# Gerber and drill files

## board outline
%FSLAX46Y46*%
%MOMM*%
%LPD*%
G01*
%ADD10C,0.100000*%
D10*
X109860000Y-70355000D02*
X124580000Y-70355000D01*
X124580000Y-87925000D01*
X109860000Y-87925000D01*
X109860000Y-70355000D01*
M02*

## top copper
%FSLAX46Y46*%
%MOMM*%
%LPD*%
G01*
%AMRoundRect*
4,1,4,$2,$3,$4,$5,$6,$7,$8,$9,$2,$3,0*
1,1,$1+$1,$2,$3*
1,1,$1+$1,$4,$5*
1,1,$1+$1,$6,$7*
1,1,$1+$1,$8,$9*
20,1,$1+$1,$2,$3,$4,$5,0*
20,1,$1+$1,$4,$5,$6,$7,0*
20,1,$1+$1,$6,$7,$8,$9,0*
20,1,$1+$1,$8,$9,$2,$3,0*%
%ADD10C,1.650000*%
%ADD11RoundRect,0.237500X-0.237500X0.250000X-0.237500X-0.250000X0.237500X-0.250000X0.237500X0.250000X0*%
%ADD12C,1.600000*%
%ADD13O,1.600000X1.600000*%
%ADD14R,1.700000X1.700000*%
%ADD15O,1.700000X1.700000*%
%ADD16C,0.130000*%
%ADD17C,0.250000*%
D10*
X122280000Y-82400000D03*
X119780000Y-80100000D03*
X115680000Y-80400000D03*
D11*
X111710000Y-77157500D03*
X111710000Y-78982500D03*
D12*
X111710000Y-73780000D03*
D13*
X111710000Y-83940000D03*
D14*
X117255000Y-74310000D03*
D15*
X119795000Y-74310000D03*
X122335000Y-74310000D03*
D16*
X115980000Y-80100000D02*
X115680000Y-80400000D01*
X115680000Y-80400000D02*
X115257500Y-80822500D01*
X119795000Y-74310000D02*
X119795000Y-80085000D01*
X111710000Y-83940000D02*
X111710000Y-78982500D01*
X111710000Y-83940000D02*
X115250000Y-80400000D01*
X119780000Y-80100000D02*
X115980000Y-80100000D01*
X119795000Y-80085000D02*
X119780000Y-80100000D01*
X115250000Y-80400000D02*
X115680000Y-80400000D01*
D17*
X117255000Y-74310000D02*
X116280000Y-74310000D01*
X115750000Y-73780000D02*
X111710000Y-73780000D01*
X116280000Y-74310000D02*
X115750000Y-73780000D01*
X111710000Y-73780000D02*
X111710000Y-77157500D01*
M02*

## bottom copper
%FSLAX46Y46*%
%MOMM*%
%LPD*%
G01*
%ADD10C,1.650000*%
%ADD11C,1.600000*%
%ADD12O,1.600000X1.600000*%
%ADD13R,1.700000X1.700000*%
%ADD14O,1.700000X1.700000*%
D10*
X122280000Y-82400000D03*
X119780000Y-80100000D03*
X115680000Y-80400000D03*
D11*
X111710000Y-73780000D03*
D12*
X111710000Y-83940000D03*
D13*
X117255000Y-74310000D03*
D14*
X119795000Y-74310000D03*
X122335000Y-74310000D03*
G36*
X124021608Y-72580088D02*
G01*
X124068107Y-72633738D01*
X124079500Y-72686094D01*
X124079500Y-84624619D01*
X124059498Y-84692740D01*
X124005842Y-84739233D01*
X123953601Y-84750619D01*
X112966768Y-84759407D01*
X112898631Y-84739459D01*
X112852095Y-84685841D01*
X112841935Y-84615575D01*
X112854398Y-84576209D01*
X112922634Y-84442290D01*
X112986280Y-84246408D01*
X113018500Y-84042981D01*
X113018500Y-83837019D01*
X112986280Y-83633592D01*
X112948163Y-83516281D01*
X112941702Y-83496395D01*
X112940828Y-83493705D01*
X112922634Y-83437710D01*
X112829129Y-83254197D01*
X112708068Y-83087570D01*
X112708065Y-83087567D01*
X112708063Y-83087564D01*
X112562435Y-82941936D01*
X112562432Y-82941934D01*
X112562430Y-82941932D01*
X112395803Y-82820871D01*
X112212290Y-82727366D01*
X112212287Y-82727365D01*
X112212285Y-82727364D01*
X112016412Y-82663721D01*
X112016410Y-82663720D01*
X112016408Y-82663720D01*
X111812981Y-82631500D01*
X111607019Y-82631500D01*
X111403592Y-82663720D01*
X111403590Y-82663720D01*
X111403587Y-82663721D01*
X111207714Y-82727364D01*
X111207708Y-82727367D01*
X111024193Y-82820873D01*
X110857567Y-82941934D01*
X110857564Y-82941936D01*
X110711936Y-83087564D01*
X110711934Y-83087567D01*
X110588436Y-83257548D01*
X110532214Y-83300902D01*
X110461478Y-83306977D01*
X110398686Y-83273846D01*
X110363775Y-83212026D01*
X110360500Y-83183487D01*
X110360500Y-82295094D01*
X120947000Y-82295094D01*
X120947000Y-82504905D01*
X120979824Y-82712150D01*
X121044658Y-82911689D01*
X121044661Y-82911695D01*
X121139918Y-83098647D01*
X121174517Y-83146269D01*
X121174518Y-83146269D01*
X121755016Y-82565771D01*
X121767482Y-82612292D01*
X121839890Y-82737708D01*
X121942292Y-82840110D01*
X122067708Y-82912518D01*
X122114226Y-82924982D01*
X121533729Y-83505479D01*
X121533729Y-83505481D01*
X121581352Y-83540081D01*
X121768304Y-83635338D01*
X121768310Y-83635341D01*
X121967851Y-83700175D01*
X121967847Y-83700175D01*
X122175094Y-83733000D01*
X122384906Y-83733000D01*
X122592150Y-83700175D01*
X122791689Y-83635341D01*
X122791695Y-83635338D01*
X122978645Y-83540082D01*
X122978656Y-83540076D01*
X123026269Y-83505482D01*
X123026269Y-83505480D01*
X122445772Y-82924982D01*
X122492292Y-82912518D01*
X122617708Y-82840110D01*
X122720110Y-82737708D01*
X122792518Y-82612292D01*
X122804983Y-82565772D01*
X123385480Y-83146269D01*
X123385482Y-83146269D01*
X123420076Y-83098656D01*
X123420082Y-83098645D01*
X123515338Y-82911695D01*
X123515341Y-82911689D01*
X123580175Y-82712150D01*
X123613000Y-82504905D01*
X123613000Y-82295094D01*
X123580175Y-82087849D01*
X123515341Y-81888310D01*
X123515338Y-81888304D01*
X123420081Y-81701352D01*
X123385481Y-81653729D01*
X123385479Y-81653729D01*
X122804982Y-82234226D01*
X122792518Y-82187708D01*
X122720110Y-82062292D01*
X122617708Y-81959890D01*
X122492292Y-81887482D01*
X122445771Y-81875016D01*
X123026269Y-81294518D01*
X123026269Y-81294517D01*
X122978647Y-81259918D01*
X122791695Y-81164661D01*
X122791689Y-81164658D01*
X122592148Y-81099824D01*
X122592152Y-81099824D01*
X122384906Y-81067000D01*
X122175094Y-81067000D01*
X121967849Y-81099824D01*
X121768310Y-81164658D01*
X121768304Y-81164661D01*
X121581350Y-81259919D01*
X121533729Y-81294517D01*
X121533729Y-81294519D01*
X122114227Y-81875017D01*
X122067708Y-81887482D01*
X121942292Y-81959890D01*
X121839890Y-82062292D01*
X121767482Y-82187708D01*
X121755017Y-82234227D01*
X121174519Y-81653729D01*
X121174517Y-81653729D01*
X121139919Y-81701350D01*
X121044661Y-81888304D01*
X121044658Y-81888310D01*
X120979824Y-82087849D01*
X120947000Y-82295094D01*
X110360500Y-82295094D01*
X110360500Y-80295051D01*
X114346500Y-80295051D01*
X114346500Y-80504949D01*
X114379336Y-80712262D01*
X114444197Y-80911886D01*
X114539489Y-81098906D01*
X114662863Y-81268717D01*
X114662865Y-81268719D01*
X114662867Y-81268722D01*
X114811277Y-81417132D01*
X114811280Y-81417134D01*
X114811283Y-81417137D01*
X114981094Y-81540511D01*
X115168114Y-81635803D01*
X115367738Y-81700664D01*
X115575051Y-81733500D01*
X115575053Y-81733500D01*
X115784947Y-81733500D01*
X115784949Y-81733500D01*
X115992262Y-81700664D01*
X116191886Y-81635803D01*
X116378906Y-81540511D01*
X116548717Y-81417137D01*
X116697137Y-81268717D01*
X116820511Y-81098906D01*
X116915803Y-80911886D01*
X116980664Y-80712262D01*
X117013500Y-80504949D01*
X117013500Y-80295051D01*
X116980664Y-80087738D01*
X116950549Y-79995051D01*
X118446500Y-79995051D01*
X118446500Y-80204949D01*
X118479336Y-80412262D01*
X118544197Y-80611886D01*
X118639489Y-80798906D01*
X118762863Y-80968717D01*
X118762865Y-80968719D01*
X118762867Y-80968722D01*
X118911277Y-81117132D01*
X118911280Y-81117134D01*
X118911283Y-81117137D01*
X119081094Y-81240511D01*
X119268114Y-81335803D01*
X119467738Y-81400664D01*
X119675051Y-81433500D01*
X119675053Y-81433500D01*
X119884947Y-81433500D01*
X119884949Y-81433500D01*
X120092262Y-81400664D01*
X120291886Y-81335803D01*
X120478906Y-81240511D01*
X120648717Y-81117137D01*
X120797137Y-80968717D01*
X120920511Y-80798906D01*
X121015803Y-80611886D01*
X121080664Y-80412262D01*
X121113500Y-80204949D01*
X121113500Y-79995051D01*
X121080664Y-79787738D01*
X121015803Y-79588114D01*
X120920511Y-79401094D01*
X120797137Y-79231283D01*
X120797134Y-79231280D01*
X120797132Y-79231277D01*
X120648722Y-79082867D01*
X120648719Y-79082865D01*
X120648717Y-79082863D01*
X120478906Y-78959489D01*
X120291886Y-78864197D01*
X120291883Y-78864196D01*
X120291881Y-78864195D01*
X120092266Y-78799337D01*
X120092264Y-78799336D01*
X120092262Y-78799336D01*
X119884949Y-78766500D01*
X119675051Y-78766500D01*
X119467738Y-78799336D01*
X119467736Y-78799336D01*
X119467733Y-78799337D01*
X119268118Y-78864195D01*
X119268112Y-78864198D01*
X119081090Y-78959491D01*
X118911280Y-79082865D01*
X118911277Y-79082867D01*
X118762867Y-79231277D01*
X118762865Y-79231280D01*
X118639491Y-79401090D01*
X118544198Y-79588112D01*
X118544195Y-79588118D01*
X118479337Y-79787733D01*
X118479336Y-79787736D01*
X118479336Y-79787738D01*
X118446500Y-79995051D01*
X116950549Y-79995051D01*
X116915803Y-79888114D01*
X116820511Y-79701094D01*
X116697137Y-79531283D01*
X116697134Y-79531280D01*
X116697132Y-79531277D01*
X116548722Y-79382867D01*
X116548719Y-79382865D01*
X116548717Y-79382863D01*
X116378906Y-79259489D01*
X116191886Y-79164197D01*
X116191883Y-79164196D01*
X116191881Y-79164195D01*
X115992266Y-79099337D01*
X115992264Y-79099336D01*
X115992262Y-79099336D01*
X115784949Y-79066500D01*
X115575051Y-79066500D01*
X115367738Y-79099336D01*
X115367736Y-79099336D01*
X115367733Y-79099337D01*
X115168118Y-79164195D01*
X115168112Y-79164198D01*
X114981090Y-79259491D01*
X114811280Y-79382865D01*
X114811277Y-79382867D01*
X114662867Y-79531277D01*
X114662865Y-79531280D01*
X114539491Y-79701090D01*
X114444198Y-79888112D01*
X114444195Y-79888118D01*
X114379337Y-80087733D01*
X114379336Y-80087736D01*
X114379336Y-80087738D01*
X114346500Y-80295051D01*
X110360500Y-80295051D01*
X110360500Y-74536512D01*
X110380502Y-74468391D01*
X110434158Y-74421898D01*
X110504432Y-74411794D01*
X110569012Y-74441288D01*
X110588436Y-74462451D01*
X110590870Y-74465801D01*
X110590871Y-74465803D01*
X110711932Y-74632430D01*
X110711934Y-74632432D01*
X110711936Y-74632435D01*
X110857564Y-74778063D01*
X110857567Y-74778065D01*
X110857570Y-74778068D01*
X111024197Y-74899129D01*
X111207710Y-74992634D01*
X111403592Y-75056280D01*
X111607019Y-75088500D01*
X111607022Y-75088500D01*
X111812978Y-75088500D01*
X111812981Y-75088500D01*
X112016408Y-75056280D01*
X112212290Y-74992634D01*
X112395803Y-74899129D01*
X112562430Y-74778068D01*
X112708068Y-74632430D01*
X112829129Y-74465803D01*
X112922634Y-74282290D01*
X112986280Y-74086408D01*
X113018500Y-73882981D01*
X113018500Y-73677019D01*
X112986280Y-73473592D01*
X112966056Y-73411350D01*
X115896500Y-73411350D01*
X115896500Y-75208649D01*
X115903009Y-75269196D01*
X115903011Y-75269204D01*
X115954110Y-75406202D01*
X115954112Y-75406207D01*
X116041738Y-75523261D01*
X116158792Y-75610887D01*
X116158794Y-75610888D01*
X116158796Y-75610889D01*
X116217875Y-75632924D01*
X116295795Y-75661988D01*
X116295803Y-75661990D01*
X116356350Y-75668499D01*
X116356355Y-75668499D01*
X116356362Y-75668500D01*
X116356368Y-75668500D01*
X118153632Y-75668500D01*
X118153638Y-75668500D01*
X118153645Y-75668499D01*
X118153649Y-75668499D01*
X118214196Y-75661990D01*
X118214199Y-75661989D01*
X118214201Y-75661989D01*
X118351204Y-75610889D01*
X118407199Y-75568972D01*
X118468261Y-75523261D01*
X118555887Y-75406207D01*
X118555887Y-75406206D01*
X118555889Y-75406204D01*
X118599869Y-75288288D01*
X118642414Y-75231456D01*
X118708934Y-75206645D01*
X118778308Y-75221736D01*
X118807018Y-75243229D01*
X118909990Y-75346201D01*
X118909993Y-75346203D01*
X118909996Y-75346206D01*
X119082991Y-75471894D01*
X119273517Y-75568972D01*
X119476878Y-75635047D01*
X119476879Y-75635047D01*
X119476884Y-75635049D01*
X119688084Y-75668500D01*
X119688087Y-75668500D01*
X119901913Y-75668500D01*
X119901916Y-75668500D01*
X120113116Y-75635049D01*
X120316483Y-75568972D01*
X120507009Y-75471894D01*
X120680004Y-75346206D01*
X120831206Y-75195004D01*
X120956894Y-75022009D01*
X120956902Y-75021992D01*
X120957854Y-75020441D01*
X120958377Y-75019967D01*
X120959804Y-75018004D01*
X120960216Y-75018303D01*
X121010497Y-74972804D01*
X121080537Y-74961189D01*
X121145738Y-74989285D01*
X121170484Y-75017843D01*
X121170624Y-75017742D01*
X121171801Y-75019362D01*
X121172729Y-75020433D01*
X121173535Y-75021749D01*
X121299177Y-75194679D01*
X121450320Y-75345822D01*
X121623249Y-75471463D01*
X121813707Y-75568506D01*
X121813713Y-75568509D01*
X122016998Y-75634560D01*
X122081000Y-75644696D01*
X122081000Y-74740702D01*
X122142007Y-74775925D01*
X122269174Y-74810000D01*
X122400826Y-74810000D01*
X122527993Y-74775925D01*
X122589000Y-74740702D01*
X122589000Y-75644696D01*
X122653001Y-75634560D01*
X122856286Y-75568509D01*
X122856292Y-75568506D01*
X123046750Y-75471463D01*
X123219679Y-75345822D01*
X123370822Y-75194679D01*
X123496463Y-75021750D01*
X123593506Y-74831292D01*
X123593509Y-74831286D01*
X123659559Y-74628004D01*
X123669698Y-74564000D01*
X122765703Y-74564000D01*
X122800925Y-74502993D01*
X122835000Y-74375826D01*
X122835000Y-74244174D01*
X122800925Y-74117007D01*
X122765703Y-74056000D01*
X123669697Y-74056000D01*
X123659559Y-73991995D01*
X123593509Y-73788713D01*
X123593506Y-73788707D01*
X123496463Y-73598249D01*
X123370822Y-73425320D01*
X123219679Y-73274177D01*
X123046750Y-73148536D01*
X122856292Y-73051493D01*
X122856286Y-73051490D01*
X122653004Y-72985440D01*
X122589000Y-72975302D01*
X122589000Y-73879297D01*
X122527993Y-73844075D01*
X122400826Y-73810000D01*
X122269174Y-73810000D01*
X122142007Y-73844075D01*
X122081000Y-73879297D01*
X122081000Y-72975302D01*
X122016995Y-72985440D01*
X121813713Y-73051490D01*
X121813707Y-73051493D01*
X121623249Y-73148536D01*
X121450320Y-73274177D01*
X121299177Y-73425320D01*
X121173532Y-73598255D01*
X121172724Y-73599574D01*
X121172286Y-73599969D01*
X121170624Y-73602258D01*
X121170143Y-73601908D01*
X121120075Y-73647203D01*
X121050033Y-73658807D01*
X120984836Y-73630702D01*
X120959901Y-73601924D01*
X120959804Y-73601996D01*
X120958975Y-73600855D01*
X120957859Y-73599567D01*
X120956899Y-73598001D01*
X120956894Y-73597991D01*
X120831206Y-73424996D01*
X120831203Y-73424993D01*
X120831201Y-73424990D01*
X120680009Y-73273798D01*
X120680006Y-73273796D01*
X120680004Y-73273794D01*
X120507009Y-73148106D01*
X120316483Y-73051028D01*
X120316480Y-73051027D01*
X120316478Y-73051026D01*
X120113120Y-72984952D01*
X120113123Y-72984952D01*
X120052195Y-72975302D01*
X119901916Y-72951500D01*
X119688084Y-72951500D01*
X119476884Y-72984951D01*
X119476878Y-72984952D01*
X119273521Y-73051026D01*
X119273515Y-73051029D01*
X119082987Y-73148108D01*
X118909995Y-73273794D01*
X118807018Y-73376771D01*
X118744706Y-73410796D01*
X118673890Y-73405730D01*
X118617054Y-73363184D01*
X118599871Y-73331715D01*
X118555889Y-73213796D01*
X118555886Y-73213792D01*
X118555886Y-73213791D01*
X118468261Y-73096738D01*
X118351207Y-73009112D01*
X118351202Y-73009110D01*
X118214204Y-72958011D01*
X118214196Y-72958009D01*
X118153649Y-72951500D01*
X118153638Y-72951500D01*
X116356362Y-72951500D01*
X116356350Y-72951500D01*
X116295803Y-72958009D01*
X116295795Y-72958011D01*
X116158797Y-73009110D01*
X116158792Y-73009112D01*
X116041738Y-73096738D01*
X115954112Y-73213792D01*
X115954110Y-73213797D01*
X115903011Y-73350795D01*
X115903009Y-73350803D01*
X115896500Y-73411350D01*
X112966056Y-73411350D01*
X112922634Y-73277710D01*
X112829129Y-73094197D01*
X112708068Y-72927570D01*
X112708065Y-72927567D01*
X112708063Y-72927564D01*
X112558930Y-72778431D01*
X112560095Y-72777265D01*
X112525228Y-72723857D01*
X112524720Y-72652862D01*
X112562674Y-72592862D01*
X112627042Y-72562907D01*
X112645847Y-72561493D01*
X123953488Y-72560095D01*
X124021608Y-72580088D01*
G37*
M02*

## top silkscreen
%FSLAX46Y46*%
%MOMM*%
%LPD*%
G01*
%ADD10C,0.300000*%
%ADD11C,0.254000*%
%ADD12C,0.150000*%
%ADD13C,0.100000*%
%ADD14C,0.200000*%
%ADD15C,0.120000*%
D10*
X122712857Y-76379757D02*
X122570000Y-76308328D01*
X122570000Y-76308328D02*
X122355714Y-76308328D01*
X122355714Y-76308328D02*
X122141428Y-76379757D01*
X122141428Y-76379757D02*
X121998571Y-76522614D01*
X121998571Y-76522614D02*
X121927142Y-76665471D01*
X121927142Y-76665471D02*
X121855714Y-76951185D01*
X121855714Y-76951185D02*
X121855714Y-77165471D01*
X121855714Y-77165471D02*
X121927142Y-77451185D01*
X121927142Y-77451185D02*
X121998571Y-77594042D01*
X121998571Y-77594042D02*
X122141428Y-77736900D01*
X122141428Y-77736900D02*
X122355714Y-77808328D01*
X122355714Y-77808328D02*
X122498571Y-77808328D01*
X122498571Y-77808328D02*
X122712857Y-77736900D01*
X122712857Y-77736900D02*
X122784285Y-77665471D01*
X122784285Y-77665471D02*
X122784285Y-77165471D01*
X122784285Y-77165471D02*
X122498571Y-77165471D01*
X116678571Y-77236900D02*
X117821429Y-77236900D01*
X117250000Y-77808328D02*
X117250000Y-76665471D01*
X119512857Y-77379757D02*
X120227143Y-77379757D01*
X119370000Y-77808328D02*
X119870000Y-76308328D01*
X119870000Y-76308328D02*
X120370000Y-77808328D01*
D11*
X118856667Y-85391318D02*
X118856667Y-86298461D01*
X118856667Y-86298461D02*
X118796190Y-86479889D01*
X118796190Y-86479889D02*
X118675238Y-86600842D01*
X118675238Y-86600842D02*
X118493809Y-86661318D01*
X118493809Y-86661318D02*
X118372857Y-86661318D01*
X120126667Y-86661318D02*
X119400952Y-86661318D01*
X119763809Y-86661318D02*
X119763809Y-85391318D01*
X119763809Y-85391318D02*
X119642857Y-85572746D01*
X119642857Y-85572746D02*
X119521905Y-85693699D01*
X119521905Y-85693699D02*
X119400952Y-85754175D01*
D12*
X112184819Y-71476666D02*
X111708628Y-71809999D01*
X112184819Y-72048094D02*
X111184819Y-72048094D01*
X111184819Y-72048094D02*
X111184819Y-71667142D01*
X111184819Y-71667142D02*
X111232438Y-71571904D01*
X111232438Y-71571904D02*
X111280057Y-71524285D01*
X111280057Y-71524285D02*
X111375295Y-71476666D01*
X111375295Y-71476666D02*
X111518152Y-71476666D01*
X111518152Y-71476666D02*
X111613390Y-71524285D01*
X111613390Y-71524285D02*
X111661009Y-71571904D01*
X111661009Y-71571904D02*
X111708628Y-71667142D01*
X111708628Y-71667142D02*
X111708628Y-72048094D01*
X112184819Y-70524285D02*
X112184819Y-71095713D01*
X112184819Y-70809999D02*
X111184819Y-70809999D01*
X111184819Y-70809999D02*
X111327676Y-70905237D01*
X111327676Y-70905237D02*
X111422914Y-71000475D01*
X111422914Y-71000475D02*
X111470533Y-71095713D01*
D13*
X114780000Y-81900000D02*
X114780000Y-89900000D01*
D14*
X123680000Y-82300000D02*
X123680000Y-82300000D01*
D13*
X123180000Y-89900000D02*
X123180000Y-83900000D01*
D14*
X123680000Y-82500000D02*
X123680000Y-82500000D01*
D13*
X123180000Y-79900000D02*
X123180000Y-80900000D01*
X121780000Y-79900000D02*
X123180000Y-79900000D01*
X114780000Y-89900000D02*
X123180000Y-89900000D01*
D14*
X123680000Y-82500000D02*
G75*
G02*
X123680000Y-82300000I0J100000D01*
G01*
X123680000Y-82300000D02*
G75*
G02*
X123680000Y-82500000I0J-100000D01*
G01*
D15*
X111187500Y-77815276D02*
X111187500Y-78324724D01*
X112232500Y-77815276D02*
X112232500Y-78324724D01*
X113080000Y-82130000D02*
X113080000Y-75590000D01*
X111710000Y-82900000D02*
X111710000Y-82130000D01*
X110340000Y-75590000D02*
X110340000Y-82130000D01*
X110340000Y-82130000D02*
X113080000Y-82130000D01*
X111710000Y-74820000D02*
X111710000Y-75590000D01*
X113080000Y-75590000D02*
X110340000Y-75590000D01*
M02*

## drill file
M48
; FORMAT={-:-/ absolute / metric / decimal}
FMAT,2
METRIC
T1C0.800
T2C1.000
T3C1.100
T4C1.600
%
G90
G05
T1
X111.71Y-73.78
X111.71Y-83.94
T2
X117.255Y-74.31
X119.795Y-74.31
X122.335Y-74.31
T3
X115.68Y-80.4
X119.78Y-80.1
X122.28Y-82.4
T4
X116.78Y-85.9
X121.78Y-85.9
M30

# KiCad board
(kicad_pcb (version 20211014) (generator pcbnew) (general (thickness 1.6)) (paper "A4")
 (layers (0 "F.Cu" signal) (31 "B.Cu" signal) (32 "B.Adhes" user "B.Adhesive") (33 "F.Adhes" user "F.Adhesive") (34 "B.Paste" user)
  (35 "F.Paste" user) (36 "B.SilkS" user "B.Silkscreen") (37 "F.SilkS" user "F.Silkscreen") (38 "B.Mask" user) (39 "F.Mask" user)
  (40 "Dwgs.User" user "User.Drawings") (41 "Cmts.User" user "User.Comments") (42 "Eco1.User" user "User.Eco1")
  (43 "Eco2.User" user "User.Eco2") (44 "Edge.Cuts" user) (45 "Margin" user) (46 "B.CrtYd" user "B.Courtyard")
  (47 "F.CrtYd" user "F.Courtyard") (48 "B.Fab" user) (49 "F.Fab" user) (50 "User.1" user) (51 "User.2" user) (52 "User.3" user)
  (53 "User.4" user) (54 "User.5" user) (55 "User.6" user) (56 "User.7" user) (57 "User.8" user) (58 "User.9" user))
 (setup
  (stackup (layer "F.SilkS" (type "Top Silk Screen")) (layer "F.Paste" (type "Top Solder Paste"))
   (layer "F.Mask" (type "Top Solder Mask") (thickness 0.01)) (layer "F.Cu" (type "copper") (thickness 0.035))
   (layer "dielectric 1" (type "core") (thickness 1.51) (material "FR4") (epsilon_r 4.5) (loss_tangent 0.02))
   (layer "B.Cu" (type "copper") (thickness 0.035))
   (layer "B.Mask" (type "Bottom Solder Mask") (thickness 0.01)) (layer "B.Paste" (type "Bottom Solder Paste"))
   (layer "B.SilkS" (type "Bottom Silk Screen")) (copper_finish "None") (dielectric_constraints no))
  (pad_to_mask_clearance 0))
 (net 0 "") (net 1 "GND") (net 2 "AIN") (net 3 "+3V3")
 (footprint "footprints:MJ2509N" (layer "F.Cu") (at 117.28 84)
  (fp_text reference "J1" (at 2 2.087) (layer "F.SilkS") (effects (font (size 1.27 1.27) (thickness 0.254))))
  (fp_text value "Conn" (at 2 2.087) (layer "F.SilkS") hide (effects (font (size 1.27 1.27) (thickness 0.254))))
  (fp_line (start -2.5 -2.1) (end -2.5 5.9) (layer "F.SilkS") (width 0.1))
  (fp_line (start 6.4 -1.7) (end 6.4 -1.7) (layer "F.SilkS") (width 0.2))
  (fp_line (start 5.9 5.9) (end 5.9 -0.1) (layer "F.SilkS") (width 0.1))
  (fp_line (start 6.4 -1.5) (end 6.4 -1.5) (layer "F.SilkS") (width 0.2))
  (fp_line (start 5.9 -4.1) (end 5.9 -3.1) (layer "F.SilkS") (width 0.1))
  (fp_line (start 4.5 -4.1) (end 5.9 -4.1) (layer "F.SilkS") (width 0.1))
  (fp_line (start -2.5 5.9) (end 5.9 5.9) (layer "F.SilkS") (width 0.1))
  (fp_arc (start 6.4 -1.5) (mid 6.3 -1.6) (end 6.4 -1.7) (layer "F.SilkS") (width 0.2))
  (fp_arc (start 6.4 -1.7) (mid 6.5 -1.6) (end 6.4 -1.5) (layer "F.SilkS") (width 0.2))
  (pad "" np_thru_hole circle (at -0.5 1.9) (size 1.6 1.6) (drill 1.6) (layers *.Cu *.Mask))
  (pad "" np_thru_hole circle (at 4.5 1.9) (size 1.6 1.6) (drill 1.6) (layers *.Cu *.Mask))
  (pad "1" thru_hole circle (at 5 -1.6) (size 1.65 1.65) (drill 1.1) (layers *.Cu *.Mask) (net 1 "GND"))
  (pad "2" thru_hole circle (at 2.5 -3.9) (size 1.65 1.65) (drill 1.1) (layers *.Cu *.Mask) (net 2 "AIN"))
  (pad "3" thru_hole circle (at -1.6 -3.6) (size 1.65 1.65) (drill 1.1) (layers *.Cu *.Mask) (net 2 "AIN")))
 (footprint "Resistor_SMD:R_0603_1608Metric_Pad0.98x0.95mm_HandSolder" (layer "F.Cu") (at 111.71 78.07 -90)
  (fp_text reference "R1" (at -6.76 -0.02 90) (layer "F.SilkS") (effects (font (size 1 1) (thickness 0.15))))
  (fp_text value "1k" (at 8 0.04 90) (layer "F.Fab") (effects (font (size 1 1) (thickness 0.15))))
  (fp_line (start -0.254724 0.5225) (end 0.254724 0.5225) (layer "F.SilkS") (width 0.12))
  (fp_line (start -0.254724 -0.5225) (end 0.254724 -0.5225) (layer "F.SilkS") (width 0.12))
  (pad "1" smd roundrect (at -0.9125 0 270) (size 0.975 0.95) (layers "F.Cu" "F.Paste" "F.Mask") (roundrect_rratio 0.25) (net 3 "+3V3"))
  (pad "2" smd roundrect (at 0.9125 0 270) (size 0.975 0.95) (layers "F.Cu" "F.Paste" "F.Mask") (roundrect_rratio 0.25) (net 2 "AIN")))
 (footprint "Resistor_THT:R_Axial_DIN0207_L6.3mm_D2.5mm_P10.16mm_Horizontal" (layer "F.Cu") (at 111.71 73.78 -90)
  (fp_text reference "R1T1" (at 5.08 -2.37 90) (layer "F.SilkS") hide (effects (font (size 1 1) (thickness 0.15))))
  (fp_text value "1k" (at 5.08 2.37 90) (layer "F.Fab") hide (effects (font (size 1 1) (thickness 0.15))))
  (fp_line (start 8.35 -1.37) (end 1.81 -1.37) (layer "F.SilkS") (width 0.12))
  (fp_line (start 9.12 0) (end 8.35 0) (layer "F.SilkS") (width 0.12))
  (fp_line (start 1.81 1.37) (end 8.35 1.37) (layer "F.SilkS") (width 0.12))
  (fp_line (start 8.35 1.37) (end 8.35 -1.37) (layer "F.SilkS") (width 0.12))
  (fp_line (start 1.04 0) (end 1.81 0) (layer "F.SilkS") (width 0.12))
  (fp_line (start 1.81 -1.37) (end 1.81 1.37) (layer "F.SilkS") (width 0.12))
  (pad "1" thru_hole circle (at 0 0 270) (size 1.6 1.6) (drill 0.8) (layers *.Cu *.Mask) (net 3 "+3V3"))
  (pad "2" thru_hole oval (at 10.16 0 270) (size 1.6 1.6) (drill 0.8) (layers *.Cu *.Mask) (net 2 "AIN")))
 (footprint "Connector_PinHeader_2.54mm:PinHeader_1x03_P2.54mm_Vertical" (layer "B.Cu") (at 117.255 74.31 -90)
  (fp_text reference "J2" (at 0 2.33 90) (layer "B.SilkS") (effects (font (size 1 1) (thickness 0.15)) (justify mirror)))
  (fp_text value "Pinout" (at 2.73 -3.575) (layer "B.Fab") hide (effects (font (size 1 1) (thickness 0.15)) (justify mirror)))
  (pad "1" thru_hole rect (at 0 0 270) (size 1.7 1.7) (drill 1) (layers *.Cu *.Mask) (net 3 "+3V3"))
  (pad "2" thru_hole oval (at 0 -2.54 270) (size 1.7 1.7) (drill 1) (layers *.Cu *.Mask) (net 2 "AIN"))
  (pad "3" thru_hole oval (at 0 -5.08 270) (size 1.7 1.7) (drill 1) (layers *.Cu *.Mask) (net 1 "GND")))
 (gr_rect (start 109.86 70.355) (end 124.58 87.925) (layer "Edge.Cuts") (width 0.1) (fill none))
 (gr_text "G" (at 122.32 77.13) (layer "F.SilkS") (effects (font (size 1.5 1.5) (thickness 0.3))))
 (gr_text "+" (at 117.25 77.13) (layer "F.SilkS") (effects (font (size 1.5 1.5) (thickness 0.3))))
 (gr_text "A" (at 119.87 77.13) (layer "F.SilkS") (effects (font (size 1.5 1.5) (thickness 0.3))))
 (segment (start 115.98 80.1) (end 115.68 80.4) (width 0.13) (layer "F.Cu") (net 2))
 (segment (start 115.68 80.4) (end 115.2575 80.8225) (width 0.13) (layer "F.Cu") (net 2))
 (segment (start 119.795 74.31) (end 119.795 80.085) (width 0.13) (layer "F.Cu") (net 2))
 (segment (start 111.71 83.94) (end 111.71 78.9825) (width 0.13) (layer "F.Cu") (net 2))
 (segment (start 111.71 83.94) (end 115.25 80.4) (width 0.13) (layer "F.Cu") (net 2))
 (segment (start 119.78 80.1) (end 115.98 80.1) (width 0.13) (layer "F.Cu") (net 2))
 (segment (start 119.795 80.085) (end 119.78 80.1) (width 0.13) (layer "F.Cu") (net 2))
 (segment (start 115.25 80.4) (end 115.68 80.4) (width 0.13) (layer "F.Cu") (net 2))
 (segment (start 117.255 74.31) (end 116.28 74.31) (width 0.25) (layer "F.Cu") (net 3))
 (segment (start 115.75 73.78) (end 111.71 73.78) (width 0.25) (layer "F.Cu") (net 3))
 (segment (start 116.28 74.31) (end 115.75 73.78) (width 0.25) (layer "F.Cu") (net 3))
 (segment (start 111.71 73.78) (end 111.71 77.1575) (width 0.25) (layer "F.Cu") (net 3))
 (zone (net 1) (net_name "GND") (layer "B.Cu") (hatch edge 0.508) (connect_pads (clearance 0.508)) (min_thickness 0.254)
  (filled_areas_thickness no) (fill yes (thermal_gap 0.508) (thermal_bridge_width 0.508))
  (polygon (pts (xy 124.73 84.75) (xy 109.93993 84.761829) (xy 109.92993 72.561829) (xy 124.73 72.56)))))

